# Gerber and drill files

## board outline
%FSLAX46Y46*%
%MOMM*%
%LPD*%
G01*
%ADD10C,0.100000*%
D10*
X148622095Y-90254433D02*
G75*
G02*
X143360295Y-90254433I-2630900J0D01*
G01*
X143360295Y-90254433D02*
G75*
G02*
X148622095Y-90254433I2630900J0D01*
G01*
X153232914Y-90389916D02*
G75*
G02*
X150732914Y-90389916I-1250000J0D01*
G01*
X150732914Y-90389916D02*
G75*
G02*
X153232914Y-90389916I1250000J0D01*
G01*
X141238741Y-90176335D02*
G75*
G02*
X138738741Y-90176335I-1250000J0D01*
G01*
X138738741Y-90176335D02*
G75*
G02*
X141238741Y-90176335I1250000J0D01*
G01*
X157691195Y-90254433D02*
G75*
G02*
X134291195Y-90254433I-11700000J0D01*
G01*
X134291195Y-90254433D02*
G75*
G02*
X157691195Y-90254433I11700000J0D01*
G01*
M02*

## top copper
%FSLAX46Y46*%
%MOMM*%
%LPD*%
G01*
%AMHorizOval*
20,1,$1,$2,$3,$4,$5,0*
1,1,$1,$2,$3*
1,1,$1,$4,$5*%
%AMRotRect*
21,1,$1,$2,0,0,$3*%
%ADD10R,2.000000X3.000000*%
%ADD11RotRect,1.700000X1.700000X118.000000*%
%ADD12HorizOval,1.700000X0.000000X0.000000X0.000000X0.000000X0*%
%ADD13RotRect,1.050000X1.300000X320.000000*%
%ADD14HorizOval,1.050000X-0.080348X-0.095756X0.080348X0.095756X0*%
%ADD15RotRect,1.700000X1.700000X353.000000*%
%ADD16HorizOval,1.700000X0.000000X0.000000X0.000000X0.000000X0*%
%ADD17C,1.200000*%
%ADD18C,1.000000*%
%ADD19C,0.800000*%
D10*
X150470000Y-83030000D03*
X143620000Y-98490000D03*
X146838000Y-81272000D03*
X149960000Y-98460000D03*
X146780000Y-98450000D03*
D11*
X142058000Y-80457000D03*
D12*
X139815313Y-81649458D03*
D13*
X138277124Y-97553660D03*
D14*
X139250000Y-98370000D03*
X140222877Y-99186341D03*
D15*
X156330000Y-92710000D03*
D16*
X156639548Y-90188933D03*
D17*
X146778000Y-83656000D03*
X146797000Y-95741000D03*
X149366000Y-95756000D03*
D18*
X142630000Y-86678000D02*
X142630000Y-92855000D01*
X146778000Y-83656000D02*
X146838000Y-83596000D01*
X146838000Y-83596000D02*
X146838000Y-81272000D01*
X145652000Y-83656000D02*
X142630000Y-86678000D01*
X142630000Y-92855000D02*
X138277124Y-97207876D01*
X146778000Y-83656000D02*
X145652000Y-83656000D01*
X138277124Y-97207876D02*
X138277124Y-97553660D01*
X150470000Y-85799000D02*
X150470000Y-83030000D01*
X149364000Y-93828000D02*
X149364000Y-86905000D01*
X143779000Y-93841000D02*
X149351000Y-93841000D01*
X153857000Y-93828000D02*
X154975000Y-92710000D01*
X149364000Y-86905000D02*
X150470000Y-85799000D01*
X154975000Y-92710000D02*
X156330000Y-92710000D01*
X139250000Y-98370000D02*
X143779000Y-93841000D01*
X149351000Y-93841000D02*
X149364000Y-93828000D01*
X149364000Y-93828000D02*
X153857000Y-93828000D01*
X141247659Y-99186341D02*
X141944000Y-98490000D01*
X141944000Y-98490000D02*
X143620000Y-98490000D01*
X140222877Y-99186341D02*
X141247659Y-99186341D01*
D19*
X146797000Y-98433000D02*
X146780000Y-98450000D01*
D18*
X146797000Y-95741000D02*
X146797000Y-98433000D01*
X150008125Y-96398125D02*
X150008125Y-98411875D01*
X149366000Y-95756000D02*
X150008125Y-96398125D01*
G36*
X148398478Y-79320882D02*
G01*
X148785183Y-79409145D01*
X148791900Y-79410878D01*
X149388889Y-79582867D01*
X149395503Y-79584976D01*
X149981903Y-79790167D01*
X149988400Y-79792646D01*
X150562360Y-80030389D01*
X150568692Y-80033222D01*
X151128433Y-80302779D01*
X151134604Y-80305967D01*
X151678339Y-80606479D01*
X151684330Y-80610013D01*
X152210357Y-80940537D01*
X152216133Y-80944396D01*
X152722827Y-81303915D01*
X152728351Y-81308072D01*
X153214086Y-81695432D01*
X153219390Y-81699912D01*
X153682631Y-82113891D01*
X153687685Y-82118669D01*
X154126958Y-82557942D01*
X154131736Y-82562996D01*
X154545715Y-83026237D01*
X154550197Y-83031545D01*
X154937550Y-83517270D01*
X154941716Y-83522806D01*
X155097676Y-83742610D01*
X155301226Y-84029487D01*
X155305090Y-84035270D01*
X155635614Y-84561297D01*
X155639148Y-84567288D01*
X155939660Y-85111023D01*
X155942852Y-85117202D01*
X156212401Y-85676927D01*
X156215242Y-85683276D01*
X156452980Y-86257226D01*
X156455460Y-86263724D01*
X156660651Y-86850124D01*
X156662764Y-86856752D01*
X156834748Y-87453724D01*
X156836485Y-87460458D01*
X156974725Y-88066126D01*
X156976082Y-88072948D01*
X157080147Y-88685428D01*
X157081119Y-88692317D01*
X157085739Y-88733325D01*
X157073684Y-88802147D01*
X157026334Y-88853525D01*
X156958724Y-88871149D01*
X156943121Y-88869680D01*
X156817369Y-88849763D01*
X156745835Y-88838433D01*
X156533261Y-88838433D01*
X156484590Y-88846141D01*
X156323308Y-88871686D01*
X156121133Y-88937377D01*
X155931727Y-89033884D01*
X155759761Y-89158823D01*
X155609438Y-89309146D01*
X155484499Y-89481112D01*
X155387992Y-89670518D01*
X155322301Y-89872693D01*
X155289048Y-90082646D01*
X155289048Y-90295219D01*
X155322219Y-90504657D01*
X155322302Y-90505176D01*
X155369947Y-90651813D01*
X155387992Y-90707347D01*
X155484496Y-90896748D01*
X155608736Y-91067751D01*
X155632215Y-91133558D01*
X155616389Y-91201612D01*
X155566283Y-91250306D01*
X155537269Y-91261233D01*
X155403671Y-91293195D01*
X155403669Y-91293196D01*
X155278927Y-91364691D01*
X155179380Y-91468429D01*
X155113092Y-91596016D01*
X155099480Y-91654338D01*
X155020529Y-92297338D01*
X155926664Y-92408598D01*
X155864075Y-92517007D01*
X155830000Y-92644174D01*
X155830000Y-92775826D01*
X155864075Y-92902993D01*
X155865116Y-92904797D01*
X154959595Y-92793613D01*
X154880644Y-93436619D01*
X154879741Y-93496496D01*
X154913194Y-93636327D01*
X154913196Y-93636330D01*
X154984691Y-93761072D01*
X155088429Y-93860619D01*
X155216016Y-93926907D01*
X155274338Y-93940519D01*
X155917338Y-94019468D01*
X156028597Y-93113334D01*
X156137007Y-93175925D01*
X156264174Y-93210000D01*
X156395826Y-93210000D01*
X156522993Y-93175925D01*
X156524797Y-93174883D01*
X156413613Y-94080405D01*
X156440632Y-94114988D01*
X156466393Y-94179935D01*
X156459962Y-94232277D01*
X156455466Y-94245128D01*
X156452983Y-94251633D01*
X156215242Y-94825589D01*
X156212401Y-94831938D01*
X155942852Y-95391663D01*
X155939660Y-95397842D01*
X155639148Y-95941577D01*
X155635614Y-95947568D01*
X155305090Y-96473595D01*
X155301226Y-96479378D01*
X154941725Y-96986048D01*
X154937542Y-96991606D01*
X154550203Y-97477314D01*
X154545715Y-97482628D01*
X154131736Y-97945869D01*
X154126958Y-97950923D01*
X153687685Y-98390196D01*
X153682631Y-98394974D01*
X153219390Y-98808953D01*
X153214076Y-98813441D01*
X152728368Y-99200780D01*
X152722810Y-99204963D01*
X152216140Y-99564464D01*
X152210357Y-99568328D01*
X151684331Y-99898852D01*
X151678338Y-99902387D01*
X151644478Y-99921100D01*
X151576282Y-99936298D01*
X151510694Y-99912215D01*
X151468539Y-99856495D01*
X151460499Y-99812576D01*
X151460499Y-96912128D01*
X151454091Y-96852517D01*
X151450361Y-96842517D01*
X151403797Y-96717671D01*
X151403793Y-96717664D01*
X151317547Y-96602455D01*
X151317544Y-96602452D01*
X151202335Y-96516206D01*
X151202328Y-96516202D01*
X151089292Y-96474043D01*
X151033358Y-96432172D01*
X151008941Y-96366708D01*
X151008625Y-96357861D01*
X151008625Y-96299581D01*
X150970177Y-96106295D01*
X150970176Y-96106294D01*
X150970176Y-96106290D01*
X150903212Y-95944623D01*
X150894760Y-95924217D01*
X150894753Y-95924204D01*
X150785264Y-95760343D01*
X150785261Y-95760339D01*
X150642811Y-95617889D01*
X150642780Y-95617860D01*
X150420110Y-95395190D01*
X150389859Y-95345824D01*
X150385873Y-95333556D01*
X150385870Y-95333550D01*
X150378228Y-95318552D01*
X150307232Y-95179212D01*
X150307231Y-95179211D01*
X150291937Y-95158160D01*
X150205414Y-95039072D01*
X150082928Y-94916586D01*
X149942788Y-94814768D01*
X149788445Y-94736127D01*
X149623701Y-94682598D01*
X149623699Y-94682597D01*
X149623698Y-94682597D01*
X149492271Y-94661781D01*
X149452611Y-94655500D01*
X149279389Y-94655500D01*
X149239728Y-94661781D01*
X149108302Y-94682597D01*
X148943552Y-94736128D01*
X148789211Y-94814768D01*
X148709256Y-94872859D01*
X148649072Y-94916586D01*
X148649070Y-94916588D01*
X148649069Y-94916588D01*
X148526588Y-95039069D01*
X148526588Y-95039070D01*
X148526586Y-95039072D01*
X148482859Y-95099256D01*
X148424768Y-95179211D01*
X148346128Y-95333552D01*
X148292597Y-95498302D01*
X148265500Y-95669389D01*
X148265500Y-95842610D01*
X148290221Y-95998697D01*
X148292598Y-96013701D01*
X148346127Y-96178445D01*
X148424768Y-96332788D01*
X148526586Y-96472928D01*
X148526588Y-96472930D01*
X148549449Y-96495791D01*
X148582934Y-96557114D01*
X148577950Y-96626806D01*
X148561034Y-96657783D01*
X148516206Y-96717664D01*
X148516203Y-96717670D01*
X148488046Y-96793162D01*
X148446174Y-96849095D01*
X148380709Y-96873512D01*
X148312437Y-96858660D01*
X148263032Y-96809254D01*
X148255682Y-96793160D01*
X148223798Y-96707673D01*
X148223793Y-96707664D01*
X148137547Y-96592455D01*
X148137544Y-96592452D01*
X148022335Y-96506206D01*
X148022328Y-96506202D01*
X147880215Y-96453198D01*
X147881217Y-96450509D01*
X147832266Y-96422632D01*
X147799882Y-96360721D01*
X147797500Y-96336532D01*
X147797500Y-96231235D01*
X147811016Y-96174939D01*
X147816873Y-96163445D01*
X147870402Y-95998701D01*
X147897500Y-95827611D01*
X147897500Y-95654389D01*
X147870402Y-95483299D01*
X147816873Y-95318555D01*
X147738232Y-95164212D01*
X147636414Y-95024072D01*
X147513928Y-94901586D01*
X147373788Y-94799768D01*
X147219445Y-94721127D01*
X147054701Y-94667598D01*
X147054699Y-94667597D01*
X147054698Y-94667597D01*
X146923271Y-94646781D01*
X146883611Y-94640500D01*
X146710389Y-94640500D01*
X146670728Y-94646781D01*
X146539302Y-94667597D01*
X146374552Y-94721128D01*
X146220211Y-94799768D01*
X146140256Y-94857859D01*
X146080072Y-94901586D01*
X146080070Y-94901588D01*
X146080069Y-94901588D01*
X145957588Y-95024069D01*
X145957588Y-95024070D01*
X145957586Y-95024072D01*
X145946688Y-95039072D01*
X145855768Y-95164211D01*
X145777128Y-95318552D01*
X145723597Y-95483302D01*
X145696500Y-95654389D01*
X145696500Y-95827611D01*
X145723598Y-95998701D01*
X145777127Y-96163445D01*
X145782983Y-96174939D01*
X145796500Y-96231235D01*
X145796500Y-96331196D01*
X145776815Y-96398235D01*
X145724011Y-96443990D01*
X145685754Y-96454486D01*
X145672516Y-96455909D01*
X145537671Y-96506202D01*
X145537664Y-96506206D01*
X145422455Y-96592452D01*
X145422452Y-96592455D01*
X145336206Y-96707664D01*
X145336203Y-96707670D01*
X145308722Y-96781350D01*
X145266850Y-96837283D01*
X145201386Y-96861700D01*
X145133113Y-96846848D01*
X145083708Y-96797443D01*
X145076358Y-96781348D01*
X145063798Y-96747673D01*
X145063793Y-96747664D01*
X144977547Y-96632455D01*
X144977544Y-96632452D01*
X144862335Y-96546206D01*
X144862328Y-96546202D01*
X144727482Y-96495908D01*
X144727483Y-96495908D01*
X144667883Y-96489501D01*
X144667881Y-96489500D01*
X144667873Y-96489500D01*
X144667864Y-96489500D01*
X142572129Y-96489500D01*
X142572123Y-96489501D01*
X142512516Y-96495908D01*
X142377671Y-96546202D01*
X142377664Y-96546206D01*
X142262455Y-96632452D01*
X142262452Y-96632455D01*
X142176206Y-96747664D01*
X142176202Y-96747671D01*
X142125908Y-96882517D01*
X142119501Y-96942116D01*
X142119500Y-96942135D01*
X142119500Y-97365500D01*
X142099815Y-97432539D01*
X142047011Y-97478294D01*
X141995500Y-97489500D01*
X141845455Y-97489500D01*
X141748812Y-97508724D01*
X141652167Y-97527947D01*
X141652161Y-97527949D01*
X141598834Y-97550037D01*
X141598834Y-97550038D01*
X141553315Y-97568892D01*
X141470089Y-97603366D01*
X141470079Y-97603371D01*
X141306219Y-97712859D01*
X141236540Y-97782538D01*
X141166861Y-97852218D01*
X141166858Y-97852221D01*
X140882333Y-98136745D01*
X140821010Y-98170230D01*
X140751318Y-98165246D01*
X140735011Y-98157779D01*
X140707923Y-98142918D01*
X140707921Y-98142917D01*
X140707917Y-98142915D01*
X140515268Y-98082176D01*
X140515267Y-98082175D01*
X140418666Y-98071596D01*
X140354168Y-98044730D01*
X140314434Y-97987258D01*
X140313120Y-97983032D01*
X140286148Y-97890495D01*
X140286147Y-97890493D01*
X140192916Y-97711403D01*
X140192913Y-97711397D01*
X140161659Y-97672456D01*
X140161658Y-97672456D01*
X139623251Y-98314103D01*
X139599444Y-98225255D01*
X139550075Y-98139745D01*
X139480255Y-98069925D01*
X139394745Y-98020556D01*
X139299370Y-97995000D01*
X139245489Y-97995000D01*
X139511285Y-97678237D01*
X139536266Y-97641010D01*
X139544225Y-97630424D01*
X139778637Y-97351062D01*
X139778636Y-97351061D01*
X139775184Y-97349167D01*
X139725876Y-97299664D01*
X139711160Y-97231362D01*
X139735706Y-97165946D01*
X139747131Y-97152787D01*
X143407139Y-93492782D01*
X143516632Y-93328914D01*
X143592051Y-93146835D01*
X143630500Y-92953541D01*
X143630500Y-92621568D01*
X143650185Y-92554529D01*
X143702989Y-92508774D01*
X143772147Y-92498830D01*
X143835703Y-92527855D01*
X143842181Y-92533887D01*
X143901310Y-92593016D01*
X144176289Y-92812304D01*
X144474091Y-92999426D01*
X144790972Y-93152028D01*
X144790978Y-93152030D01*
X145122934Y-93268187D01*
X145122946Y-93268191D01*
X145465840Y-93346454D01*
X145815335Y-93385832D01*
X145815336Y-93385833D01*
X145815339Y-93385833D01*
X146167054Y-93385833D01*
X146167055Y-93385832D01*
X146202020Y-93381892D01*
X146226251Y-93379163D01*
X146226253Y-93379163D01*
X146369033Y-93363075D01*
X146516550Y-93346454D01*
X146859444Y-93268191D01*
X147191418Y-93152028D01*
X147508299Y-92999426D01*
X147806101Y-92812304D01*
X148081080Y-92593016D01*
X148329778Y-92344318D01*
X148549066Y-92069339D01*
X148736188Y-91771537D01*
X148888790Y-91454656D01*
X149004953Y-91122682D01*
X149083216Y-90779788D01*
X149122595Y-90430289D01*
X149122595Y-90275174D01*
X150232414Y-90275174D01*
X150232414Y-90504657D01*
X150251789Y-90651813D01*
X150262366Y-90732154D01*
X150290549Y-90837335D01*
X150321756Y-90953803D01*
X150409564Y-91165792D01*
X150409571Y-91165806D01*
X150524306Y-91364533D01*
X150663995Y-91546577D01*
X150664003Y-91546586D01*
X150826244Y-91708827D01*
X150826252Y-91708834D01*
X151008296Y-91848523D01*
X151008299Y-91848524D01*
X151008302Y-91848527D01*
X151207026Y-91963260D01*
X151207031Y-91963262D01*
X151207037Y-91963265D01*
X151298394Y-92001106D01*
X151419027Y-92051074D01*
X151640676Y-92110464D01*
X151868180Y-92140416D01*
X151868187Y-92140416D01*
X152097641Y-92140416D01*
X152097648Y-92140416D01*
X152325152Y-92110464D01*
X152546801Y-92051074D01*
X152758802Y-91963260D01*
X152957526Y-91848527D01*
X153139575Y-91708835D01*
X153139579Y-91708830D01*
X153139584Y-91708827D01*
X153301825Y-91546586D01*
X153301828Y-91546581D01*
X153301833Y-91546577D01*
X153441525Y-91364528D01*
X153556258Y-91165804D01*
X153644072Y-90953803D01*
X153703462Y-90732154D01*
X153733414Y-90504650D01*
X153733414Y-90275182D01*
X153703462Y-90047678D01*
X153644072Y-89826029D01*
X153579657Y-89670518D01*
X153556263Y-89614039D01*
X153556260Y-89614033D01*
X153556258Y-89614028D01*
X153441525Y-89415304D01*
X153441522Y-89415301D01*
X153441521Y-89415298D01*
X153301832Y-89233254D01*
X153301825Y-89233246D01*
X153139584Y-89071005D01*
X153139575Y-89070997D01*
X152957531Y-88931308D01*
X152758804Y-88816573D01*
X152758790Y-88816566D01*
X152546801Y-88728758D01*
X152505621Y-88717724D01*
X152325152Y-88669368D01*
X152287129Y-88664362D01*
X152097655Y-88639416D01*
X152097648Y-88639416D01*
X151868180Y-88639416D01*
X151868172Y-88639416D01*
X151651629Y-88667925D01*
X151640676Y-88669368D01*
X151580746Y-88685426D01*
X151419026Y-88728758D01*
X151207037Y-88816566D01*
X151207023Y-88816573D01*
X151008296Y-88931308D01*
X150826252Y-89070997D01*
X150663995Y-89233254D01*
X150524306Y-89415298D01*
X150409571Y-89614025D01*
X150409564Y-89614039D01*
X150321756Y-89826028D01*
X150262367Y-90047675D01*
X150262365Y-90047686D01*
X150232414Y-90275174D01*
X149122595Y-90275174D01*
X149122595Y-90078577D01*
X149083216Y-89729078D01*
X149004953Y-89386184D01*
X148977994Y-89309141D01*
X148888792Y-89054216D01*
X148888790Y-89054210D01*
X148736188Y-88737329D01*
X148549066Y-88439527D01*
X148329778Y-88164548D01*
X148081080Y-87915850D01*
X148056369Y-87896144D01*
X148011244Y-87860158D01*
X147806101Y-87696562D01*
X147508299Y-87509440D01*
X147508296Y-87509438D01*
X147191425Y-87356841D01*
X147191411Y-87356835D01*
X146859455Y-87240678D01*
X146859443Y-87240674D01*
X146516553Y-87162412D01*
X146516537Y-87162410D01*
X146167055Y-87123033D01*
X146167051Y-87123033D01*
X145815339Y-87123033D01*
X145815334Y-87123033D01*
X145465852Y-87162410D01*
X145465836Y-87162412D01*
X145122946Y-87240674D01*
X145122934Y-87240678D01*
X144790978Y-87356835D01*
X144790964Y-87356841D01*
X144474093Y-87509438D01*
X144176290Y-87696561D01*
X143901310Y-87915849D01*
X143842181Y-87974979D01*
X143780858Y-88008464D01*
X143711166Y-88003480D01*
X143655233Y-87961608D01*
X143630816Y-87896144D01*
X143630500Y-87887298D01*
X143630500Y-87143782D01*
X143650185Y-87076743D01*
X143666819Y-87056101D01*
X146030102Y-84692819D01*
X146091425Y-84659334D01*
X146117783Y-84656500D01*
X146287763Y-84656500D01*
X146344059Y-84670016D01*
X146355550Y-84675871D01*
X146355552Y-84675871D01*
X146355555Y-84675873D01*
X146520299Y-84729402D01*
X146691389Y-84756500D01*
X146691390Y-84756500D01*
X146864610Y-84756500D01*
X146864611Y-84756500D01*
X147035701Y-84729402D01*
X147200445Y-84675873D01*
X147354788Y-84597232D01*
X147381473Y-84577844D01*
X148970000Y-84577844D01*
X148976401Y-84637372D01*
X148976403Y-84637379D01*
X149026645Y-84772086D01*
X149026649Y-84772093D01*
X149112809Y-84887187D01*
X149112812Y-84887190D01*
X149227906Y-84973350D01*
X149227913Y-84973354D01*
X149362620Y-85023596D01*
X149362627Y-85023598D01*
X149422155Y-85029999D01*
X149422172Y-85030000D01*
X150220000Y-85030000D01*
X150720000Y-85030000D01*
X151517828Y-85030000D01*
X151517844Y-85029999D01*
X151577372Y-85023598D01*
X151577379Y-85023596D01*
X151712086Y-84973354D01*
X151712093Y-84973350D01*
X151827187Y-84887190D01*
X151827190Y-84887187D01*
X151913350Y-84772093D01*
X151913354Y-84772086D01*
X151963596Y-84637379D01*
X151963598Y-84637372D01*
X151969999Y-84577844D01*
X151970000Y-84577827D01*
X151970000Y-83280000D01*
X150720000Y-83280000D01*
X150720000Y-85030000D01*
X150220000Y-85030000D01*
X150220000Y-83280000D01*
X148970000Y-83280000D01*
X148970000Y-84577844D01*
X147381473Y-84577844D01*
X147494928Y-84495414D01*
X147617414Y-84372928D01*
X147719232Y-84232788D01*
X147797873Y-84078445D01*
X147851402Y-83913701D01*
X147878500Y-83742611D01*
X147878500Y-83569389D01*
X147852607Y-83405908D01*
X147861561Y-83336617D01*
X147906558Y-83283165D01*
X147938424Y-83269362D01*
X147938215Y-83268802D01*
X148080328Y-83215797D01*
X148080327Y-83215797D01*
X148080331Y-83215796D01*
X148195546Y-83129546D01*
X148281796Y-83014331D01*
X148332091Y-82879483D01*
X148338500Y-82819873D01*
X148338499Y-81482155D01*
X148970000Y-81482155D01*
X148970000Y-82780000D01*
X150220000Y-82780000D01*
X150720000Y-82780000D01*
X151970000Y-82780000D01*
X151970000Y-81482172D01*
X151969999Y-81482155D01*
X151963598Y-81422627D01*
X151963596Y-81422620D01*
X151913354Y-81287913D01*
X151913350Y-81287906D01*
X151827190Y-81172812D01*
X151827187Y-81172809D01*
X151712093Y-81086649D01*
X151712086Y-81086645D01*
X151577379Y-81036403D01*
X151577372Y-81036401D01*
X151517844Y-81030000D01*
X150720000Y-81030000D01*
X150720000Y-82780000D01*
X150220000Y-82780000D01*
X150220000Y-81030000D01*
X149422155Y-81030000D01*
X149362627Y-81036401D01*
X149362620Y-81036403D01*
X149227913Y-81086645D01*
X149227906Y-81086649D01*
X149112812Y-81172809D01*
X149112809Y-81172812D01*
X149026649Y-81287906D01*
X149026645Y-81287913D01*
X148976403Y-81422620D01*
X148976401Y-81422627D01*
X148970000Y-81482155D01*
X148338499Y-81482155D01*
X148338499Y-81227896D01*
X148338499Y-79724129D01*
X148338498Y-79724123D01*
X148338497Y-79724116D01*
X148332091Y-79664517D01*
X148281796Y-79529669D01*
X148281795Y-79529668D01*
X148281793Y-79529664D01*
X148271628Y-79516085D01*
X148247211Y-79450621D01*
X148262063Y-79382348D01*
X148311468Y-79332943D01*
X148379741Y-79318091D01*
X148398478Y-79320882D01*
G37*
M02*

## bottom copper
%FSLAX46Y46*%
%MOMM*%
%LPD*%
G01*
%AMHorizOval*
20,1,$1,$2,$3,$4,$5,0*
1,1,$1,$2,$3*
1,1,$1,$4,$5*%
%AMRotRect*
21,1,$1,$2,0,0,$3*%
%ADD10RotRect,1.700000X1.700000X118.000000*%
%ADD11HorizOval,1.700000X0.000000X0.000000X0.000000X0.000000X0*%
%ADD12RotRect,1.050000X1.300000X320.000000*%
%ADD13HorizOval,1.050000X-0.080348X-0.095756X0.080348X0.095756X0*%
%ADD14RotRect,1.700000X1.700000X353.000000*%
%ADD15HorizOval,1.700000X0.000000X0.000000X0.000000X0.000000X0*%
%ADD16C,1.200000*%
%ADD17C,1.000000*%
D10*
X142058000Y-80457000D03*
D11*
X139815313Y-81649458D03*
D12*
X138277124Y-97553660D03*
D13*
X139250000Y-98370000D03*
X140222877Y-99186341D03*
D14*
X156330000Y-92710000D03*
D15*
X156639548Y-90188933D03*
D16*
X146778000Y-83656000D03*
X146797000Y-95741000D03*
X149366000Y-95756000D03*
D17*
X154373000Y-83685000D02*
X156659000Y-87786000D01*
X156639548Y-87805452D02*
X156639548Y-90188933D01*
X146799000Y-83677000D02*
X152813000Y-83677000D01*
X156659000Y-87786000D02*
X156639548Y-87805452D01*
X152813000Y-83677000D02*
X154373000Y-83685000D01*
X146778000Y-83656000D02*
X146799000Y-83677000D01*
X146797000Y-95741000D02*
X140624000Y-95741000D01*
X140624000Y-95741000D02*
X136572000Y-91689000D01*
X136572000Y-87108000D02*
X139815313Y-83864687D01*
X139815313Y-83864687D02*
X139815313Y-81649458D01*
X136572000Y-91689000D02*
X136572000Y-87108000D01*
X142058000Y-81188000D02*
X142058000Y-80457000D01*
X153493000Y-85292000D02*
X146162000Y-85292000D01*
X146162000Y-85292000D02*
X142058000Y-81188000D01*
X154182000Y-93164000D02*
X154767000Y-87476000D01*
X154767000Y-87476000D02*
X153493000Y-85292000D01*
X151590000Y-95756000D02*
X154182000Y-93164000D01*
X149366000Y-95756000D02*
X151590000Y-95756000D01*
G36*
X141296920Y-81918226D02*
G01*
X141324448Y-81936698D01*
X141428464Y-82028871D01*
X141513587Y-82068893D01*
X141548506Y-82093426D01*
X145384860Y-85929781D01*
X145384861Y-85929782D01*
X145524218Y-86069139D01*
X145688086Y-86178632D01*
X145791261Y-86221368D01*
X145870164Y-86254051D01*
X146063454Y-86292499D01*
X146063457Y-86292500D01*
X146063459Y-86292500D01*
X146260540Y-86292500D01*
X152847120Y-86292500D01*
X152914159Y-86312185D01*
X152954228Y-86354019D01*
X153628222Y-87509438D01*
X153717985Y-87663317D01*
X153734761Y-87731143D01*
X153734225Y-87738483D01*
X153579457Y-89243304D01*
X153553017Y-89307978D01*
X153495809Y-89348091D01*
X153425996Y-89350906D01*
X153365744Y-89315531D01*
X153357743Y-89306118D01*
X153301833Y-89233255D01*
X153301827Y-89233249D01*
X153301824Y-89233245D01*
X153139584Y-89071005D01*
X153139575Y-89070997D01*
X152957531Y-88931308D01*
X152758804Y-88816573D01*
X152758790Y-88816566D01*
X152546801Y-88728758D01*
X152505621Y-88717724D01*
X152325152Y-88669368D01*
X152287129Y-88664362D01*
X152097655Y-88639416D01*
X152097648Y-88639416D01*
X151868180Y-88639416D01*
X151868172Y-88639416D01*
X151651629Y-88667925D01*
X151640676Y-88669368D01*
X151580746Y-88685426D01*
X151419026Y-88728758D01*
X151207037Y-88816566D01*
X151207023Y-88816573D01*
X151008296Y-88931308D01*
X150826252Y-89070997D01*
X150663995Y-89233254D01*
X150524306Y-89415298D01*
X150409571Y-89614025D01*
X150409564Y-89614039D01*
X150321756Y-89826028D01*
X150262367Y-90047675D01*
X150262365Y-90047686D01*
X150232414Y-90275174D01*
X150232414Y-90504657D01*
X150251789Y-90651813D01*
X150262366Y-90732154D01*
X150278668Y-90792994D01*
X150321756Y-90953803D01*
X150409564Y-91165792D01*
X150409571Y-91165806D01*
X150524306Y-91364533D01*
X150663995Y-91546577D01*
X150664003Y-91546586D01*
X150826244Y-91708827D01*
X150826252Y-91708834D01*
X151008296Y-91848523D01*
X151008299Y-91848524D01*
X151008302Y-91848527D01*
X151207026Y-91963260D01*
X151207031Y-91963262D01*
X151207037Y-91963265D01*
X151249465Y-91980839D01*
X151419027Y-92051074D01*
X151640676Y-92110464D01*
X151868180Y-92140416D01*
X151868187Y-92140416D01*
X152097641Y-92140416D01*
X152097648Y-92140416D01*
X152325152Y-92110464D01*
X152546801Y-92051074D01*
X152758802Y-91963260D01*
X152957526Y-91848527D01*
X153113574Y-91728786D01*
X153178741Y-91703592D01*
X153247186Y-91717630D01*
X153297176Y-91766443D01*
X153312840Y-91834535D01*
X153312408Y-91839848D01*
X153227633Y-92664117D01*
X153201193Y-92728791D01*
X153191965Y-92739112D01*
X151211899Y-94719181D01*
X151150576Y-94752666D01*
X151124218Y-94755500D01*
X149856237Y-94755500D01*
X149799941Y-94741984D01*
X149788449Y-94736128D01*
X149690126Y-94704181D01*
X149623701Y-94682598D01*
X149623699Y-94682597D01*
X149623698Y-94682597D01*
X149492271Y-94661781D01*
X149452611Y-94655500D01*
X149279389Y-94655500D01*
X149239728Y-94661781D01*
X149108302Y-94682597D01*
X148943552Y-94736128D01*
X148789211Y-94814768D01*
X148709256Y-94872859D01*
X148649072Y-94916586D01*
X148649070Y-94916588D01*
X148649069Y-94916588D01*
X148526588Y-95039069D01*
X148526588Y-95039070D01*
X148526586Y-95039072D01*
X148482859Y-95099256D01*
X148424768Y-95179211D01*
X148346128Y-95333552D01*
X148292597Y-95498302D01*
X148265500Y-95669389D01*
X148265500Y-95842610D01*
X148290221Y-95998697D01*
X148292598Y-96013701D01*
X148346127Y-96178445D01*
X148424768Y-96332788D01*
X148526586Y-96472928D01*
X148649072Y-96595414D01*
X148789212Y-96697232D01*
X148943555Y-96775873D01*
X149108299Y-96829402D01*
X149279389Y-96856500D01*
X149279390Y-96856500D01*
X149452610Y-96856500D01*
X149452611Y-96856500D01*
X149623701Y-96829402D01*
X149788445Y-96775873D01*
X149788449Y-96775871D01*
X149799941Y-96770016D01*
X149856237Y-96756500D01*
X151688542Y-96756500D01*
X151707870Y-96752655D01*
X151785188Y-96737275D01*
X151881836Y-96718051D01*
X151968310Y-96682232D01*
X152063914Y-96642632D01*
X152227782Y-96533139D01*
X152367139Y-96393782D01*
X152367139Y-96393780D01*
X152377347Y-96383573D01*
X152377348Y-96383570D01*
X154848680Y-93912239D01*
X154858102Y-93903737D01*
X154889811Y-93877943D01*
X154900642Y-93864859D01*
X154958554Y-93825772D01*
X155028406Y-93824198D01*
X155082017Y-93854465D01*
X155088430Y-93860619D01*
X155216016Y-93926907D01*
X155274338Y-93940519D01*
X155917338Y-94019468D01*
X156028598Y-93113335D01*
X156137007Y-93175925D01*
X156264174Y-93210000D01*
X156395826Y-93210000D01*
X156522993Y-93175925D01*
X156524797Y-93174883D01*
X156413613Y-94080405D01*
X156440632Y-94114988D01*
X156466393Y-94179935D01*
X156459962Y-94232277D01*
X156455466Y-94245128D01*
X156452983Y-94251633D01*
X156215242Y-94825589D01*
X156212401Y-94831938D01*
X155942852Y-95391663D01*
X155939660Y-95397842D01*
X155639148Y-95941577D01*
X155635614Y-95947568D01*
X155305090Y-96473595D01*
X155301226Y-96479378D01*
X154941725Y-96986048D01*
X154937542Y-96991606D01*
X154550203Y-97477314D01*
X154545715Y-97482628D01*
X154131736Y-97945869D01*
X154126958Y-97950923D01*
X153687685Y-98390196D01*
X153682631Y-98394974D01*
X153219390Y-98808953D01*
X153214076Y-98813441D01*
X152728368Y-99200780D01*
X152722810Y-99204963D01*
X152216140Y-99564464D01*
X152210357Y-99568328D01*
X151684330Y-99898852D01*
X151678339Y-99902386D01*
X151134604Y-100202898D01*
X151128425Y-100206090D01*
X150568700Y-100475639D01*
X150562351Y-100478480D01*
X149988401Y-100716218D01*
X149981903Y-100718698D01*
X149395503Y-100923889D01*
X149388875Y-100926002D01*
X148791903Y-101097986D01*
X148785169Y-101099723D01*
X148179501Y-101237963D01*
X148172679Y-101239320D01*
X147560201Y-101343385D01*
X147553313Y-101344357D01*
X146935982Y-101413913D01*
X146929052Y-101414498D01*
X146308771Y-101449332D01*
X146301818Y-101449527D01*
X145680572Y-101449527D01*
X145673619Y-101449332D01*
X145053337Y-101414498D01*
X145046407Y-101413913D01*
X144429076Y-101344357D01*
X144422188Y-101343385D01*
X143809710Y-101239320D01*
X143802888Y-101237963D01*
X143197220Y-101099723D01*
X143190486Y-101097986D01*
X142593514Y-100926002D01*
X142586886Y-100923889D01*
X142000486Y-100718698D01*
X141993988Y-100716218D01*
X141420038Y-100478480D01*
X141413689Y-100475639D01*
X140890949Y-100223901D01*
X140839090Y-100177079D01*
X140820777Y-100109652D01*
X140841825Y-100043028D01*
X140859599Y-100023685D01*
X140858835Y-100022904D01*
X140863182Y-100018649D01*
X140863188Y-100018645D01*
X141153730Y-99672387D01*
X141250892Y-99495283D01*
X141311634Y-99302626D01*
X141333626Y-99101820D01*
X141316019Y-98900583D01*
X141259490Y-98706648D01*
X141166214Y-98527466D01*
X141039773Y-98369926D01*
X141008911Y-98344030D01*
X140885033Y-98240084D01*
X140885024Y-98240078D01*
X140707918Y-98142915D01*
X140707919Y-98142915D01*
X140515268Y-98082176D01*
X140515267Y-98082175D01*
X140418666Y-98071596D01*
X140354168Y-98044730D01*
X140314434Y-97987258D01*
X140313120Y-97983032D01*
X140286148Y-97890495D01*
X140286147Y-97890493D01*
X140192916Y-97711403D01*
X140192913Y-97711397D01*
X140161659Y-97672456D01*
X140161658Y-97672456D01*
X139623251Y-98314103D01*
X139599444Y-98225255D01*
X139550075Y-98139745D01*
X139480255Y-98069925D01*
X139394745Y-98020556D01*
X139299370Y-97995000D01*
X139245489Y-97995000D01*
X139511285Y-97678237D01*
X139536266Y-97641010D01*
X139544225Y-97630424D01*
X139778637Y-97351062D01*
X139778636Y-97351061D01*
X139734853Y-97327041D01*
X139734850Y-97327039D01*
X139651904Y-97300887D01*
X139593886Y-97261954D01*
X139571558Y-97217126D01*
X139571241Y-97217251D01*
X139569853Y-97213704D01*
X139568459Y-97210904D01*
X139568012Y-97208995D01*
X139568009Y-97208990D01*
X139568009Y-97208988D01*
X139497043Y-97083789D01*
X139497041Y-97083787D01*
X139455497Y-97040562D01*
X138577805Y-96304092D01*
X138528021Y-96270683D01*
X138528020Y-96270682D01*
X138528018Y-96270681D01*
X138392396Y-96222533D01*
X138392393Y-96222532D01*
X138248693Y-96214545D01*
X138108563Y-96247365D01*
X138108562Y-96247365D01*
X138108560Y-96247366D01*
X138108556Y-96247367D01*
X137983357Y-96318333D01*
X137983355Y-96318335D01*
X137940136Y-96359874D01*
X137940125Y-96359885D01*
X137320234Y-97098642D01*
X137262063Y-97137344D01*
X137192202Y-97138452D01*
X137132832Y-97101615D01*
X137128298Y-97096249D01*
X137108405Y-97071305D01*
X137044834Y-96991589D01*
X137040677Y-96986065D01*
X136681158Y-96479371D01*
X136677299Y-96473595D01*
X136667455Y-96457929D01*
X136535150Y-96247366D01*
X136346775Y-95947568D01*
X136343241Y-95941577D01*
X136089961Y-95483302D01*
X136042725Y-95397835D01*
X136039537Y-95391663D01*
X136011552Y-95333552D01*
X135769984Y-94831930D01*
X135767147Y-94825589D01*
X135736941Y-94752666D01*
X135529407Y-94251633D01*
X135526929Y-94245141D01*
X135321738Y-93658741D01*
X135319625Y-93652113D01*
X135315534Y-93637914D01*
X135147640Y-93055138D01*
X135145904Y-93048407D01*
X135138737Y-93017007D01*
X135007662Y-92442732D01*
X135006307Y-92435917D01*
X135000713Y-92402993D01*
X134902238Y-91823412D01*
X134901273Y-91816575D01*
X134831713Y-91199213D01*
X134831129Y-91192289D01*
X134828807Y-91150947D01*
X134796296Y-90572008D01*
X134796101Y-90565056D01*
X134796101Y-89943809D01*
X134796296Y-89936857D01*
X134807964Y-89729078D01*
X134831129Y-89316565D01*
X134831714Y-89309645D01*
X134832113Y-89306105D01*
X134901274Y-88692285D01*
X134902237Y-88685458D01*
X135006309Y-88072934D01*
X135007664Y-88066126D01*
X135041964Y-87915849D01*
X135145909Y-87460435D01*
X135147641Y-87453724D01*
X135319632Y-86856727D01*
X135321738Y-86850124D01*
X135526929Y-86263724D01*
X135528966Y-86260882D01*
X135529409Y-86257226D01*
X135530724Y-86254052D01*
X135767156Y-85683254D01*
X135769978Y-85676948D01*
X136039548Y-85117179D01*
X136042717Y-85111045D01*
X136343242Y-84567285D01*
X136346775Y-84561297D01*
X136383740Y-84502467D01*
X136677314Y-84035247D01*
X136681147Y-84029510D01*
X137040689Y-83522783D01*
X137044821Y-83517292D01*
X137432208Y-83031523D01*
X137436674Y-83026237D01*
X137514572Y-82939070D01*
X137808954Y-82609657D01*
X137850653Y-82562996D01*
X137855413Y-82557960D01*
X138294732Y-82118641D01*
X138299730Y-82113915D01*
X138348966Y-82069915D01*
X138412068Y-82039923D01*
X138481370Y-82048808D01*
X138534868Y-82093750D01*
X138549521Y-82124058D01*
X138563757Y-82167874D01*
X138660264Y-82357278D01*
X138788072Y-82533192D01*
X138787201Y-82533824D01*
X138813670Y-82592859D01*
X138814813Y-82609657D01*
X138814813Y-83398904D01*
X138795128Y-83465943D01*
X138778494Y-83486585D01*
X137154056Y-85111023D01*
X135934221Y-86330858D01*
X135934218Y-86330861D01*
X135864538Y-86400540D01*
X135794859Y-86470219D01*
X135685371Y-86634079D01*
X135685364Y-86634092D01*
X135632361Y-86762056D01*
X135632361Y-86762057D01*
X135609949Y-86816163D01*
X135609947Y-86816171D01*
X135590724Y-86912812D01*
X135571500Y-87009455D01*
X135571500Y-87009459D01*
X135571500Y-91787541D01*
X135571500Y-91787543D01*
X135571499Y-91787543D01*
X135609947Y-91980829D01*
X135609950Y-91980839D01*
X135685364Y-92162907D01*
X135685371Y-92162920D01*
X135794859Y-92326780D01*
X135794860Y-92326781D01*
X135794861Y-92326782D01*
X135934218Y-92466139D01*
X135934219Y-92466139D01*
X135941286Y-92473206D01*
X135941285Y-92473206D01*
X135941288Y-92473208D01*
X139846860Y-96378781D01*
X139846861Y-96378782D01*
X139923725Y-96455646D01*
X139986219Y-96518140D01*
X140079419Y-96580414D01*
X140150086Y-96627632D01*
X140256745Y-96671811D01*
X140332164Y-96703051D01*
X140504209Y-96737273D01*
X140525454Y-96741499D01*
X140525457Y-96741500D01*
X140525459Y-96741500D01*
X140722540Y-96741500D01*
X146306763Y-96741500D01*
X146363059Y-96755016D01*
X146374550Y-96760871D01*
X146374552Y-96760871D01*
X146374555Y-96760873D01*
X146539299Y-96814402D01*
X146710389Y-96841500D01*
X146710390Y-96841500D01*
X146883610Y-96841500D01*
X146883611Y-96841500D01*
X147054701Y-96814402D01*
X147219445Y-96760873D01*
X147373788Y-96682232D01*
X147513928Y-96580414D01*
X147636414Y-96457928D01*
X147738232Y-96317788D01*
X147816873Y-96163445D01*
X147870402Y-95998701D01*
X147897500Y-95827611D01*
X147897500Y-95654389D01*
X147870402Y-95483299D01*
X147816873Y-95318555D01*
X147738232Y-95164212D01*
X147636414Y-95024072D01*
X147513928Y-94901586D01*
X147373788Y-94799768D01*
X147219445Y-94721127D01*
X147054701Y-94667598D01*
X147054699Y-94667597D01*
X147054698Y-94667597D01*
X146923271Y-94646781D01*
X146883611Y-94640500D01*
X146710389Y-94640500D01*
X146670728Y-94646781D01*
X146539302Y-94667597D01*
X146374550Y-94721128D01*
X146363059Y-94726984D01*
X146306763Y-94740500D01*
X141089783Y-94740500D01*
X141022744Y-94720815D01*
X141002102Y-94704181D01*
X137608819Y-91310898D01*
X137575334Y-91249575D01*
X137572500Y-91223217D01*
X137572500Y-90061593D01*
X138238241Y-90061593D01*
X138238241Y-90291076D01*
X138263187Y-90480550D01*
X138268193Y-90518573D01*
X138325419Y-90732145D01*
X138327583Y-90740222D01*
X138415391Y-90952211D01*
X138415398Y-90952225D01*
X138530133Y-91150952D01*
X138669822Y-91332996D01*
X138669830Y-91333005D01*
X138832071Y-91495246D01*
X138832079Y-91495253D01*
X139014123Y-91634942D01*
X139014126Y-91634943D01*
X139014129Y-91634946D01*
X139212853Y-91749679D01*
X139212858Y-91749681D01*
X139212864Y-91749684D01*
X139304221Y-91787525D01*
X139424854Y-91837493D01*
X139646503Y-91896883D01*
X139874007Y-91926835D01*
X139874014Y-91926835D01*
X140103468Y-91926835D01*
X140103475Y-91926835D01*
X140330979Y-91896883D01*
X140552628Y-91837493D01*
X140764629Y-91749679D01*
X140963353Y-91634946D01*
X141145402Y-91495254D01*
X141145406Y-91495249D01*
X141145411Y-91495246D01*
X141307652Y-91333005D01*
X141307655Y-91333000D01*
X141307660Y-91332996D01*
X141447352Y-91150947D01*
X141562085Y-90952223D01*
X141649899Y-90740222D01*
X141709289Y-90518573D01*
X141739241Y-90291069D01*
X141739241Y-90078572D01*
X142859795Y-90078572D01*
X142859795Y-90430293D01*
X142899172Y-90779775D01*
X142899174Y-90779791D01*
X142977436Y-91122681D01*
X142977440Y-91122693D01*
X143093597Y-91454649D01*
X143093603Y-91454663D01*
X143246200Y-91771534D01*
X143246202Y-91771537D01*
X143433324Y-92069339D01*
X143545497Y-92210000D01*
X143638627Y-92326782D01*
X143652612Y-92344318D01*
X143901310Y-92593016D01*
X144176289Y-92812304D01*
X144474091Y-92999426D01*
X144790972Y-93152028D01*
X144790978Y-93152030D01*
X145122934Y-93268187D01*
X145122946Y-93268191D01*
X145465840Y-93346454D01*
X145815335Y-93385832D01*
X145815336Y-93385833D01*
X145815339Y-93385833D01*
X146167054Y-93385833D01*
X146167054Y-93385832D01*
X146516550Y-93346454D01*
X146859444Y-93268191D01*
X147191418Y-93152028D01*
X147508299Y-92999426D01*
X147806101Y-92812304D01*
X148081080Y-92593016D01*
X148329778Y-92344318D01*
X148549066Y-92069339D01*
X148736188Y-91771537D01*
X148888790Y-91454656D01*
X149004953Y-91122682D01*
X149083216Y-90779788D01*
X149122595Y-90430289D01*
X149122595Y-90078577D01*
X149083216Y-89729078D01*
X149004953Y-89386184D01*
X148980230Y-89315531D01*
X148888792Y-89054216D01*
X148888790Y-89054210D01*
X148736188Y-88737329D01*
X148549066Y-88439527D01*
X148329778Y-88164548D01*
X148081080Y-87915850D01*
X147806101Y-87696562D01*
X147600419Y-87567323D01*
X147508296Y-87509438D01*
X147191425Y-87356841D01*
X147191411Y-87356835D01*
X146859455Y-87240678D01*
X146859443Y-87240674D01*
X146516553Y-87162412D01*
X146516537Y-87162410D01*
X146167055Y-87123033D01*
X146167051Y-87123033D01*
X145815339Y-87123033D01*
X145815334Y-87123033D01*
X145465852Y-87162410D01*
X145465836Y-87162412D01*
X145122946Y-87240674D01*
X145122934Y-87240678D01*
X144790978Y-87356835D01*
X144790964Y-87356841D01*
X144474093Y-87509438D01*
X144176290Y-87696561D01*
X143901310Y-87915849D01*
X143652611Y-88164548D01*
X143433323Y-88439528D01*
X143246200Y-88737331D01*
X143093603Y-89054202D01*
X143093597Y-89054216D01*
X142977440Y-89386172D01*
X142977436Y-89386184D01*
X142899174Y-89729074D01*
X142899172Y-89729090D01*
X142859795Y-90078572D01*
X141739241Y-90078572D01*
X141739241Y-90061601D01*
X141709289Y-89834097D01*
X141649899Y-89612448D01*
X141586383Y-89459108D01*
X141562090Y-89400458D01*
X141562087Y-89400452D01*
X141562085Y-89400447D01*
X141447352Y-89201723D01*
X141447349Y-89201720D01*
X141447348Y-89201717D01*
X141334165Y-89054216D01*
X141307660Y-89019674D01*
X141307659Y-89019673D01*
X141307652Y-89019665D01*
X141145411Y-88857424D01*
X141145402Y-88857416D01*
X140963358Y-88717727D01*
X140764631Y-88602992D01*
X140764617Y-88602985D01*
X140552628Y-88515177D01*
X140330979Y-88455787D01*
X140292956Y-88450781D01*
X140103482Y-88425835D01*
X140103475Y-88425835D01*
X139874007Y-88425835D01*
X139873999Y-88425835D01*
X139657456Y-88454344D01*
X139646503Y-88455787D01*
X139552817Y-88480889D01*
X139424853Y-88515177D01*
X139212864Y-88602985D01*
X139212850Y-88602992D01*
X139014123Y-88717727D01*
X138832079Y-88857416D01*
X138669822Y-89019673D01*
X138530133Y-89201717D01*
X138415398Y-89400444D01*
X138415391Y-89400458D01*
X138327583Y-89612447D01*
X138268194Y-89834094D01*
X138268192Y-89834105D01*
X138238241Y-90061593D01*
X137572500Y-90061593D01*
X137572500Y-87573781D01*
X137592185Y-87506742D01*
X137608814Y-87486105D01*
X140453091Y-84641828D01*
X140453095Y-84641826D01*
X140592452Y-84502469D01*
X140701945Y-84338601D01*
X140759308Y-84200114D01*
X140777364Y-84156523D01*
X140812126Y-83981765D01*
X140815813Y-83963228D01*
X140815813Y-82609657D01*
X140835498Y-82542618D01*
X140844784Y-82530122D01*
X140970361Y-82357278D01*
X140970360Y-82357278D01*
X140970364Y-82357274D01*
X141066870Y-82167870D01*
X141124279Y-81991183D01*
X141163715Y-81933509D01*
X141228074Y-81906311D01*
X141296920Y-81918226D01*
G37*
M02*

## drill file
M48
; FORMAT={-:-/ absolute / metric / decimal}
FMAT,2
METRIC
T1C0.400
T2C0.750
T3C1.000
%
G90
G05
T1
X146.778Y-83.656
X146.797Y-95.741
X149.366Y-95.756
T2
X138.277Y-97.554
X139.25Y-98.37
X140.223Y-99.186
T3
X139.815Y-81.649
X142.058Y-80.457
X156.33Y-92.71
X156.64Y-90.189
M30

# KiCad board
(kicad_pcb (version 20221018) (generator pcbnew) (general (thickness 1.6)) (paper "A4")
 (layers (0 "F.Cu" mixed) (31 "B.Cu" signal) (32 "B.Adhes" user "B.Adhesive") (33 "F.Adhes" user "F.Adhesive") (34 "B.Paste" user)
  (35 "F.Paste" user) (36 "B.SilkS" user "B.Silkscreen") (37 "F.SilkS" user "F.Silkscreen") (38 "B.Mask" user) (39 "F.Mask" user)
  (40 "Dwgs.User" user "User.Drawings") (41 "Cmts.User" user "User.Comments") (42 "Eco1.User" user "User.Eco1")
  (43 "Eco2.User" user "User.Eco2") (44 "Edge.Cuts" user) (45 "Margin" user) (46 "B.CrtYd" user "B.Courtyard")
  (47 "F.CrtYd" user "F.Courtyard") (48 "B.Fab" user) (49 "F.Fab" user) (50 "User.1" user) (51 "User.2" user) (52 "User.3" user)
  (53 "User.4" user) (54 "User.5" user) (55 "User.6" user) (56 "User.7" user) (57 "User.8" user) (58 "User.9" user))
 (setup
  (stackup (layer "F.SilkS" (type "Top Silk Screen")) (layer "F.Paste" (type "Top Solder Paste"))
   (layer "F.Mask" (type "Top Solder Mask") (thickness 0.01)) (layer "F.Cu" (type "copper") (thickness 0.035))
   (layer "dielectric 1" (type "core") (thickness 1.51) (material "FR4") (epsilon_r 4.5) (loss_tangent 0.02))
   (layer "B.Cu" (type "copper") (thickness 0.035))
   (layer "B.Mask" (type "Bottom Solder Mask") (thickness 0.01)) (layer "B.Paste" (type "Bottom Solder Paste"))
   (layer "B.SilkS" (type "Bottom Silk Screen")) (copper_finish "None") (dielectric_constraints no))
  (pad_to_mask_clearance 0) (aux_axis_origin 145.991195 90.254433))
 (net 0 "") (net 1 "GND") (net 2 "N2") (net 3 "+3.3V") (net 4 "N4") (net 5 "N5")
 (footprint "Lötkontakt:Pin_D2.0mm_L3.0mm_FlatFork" (layer "F.Cu") (at 150.47 83.03)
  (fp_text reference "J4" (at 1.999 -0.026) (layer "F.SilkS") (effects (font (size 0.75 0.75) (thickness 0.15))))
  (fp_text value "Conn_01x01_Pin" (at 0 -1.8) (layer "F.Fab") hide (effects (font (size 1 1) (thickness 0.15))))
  (pad "1" connect rect (at 0 0 180) (size 2 3) (layers "F.Cu" "F.Mask") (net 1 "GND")))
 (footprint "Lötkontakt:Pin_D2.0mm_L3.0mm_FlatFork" (layer "F.Cu") (at 143.62 98.49)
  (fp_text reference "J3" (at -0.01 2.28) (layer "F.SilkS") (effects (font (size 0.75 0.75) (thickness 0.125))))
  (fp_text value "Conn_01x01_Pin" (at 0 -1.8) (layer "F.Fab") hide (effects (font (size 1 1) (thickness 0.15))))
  (pad "1" connect rect (at 0 0 180) (size 2 3) (layers "F.Cu" "F.Mask") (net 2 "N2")))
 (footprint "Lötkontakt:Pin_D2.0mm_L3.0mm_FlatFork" (layer "F.Cu") (at 146.838 81.272)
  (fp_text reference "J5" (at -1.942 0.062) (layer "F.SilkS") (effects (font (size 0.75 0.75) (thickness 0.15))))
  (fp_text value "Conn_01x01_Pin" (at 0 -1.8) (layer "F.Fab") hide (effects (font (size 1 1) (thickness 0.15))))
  (pad "1" connect rect (at 0 0 180) (size 2 3) (layers "F.Cu" "F.Mask") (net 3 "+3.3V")))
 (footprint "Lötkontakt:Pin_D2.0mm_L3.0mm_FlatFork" (layer "F.Cu") (at 149.96 98.46)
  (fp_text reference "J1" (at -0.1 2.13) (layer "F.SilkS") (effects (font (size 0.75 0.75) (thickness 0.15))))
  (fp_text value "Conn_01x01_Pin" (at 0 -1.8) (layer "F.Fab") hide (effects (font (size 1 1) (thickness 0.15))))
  (pad "1" connect rect (at 0 0 180) (size 2 3) (layers "F.Cu" "F.Mask") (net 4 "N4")))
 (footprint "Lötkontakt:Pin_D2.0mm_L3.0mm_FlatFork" (layer "F.Cu") (at 146.78 98.45)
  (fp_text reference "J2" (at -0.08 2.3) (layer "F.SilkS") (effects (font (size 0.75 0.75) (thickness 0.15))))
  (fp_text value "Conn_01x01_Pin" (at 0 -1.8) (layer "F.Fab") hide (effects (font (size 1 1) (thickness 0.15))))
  (pad "1" connect rect (at 0 0 180) (size 2 3) (layers "F.Cu" "F.Mask") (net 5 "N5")))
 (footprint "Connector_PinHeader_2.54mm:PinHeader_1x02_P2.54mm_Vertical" (layer "B.Cu") (at 142.058 80.457 118)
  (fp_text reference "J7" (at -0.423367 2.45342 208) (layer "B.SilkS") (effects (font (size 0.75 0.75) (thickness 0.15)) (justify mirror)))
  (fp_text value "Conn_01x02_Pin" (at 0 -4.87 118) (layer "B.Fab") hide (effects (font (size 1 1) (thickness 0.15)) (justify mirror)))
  (pad "1" thru_hole rect (at 0 0 118) (size 1.7 1.7) (drill 1) (layers "*.Cu" "*.Mask") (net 4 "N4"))
  (pad "2" thru_hole oval (at 0 -2.54 118) (size 1.7 1.7) (drill 1) (layers "*.Cu" "*.Mask") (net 5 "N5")))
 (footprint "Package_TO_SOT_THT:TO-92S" (layer "B.Cu") (at 138.277124 97.55366 -40)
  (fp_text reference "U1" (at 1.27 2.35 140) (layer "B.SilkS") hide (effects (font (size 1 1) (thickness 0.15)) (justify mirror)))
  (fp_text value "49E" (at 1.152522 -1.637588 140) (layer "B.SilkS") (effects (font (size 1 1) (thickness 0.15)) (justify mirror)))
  (pad "1" thru_hole rect (at 0 0 320) (size 1.05 1.3) (drill 0.75) (layers "*.Cu" "*.Mask") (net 3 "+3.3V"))
  (pad "2" thru_hole oval (at 1.27 0 320) (size 1.05 1.3) (drill 0.75) (layers "*.Cu" "*.Mask") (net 1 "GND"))
  (pad "3" thru_hole oval (at 2.54 0 320) (size 1.05 1.3) (drill 0.75) (layers "*.Cu" "*.Mask") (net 2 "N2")))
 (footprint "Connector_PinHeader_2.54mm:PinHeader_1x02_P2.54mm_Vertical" (layer "B.Cu") (at 156.33 92.71 -7)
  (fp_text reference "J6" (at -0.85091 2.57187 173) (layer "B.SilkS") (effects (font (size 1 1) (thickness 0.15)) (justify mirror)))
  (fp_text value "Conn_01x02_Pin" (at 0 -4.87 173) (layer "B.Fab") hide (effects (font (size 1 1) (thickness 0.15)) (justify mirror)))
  (pad "1" thru_hole rect (at 0 0 353) (size 1.7 1.7) (drill 1) (layers "*.Cu" "*.Mask") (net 1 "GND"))
  (pad "2" thru_hole oval (at 0 -2.54 353) (size 1.7 1.7) (drill 1) (layers "*.Cu" "*.Mask") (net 3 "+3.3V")))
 (gr_circle (center 145.991195 90.254433) (end 148.575 90.75) (stroke (width 0.1) (type default)) (fill none) (layer "Edge.Cuts"))
 (gr_circle (center 151.982914 90.389916) (end 153.232914 90.389916) (stroke (width 0.1) (type default)) (fill none) (layer "Edge.Cuts"))
 (gr_circle (center 139.988741 90.176335) (end 141.238741 90.176335) (stroke (width 0.1) (type default)) (fill none) (layer "Edge.Cuts"))
 (gr_circle (center 145.991195 90.254433) (end 157.691195 90.254433) (stroke (width 0.1) (type default)) (fill none) (layer "Edge.Cuts"))
 (segment (start 142.63 86.678) (end 142.63 92.855) (width 1) (layer "F.Cu") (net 3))
 (segment (start 146.778 83.656) (end 146.838 83.596) (width 1) (layer "F.Cu") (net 3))
 (segment (start 146.838 83.596) (end 146.838 81.272) (width 1) (layer "F.Cu") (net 3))
 (segment (start 145.652 83.656) (end 142.63 86.678) (width 1) (layer "F.Cu") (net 3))
 (segment (start 142.63 92.855) (end 138.277124 97.207876) (width 1) (layer "F.Cu") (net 3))
 (segment (start 146.778 83.656) (end 145.652 83.656) (width 1) (layer "F.Cu") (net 3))
 (segment (start 138.277124 97.207876) (end 138.277124 97.55366) (width 1) (layer "F.Cu") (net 3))
 (via (at 146.778 83.656) (size 1.2) (drill 0.4) (layers "F.Cu" "B.Cu") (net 3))
 (segment (start 154.373 83.685) (end 156.659 87.786) (width 1) (layer "B.Cu") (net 3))
 (segment (start 156.639548 87.805452) (end 156.639548 90.188933) (width 1) (layer "B.Cu") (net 3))
 (segment (start 146.799 83.677) (end 152.813 83.677) (width 1) (layer "B.Cu") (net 3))
 (segment (start 156.659 87.786) (end 156.639548 87.805452) (width 1) (layer "B.Cu") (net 3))
 (segment (start 152.813 83.677) (end 154.373 83.685) (width 1) (layer "B.Cu") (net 3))
 (segment (start 146.778 83.656) (end 146.799 83.677) (width 1) (layer "B.Cu") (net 3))
 (segment (start 150.47 85.799) (end 150.47 83.03) (width 1) (layer "F.Cu") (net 1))
 (segment (start 149.364 93.828) (end 149.364 86.905) (width 1) (layer "F.Cu") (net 1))
 (segment (start 143.779 93.841) (end 149.351 93.841) (width 1) (layer "F.Cu") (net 1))
 (segment (start 153.857 93.828) (end 154.975 92.71) (width 1) (layer "F.Cu") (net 1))
 (segment (start 149.364 86.905) (end 150.47 85.799) (width 1) (layer "F.Cu") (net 1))
 (segment (start 154.975 92.71) (end 156.33 92.71) (width 1) (layer "F.Cu") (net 1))
 (segment (start 139.25 98.37) (end 143.779 93.841) (width 1) (layer "F.Cu") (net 1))
 (segment (start 149.351 93.841) (end 149.364 93.828) (width 1) (layer "F.Cu") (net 1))
 (segment (start 149.364 93.828) (end 153.857 93.828) (width 1) (layer "F.Cu") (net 1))
 (segment (start 141.247659 99.186341) (end 141.944 98.49) (width 1) (layer "F.Cu") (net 2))
 (segment (start 141.944 98.49) (end 143.62 98.49) (width 1) (layer "F.Cu") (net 2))
 (segment (start 140.222877 99.186341) (end 141.247659 99.186341) (width 1) (layer "F.Cu") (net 2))
 (segment (start 146.797 98.433) (end 146.78 98.45) (width 0.8) (layer "F.Cu") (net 5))
 (segment (start 146.797 95.741) (end 146.797 98.433) (width 1) (layer "F.Cu") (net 5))
 (via (at 146.797 95.741) (size 1.2) (drill 0.4) (layers "F.Cu" "B.Cu") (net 5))
 (segment (start 146.797 95.741) (end 140.624 95.741) (width 1) (layer "B.Cu") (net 5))
 (segment (start 140.624 95.741) (end 136.572 91.689) (width 1) (layer "B.Cu") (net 5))
 (segment (start 136.572 87.108) (end 139.815313 83.864687) (width 1) (layer "B.Cu") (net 5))
 (segment (start 139.815313 83.864687) (end 139.815313 81.649458) (width 1) (layer "B.Cu") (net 5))
 (segment (start 136.572 91.689) (end 136.572 87.108) (width 1) (layer "B.Cu") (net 5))
 (segment (start 150.008125 96.398125) (end 150.008125 98.411875) (width 1) (layer "F.Cu") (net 4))
 (segment (start 149.366 95.756) (end 150.008125 96.398125) (width 1) (layer "F.Cu") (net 4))
 (via (at 149.366 95.756) (size 1.2) (drill 0.4) (layers "F.Cu" "B.Cu") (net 4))
 (segment (start 142.058 81.188) (end 142.058 80.457) (width 1) (layer "B.Cu") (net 4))
 (segment (start 153.493 85.292) (end 146.162 85.292) (width 1) (layer "B.Cu") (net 4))
 (segment (start 146.162 85.292) (end 142.058 81.188) (width 1) (layer "B.Cu") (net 4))
 (segment (start 154.182 93.164) (end 154.767 87.476) (width 1) (layer "B.Cu") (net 4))
 (segment (start 154.767 87.476) (end 153.493 85.292) (width 1) (layer "B.Cu") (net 4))
 (segment (start 151.59 95.756) (end 154.182 93.164) (width 1) (layer "B.Cu") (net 4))
 (segment (start 149.366 95.756) (end 151.59 95.756) (width 1) (layer "B.Cu") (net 4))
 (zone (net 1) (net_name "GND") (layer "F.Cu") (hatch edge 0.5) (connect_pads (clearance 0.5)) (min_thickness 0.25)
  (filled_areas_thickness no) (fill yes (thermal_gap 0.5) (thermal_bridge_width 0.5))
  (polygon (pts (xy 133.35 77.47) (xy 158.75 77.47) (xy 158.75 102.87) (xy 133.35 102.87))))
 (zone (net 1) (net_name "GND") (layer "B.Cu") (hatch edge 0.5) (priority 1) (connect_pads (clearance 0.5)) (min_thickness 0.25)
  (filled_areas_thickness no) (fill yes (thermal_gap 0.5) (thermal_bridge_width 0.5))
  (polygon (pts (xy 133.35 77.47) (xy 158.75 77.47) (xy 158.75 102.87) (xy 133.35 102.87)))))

